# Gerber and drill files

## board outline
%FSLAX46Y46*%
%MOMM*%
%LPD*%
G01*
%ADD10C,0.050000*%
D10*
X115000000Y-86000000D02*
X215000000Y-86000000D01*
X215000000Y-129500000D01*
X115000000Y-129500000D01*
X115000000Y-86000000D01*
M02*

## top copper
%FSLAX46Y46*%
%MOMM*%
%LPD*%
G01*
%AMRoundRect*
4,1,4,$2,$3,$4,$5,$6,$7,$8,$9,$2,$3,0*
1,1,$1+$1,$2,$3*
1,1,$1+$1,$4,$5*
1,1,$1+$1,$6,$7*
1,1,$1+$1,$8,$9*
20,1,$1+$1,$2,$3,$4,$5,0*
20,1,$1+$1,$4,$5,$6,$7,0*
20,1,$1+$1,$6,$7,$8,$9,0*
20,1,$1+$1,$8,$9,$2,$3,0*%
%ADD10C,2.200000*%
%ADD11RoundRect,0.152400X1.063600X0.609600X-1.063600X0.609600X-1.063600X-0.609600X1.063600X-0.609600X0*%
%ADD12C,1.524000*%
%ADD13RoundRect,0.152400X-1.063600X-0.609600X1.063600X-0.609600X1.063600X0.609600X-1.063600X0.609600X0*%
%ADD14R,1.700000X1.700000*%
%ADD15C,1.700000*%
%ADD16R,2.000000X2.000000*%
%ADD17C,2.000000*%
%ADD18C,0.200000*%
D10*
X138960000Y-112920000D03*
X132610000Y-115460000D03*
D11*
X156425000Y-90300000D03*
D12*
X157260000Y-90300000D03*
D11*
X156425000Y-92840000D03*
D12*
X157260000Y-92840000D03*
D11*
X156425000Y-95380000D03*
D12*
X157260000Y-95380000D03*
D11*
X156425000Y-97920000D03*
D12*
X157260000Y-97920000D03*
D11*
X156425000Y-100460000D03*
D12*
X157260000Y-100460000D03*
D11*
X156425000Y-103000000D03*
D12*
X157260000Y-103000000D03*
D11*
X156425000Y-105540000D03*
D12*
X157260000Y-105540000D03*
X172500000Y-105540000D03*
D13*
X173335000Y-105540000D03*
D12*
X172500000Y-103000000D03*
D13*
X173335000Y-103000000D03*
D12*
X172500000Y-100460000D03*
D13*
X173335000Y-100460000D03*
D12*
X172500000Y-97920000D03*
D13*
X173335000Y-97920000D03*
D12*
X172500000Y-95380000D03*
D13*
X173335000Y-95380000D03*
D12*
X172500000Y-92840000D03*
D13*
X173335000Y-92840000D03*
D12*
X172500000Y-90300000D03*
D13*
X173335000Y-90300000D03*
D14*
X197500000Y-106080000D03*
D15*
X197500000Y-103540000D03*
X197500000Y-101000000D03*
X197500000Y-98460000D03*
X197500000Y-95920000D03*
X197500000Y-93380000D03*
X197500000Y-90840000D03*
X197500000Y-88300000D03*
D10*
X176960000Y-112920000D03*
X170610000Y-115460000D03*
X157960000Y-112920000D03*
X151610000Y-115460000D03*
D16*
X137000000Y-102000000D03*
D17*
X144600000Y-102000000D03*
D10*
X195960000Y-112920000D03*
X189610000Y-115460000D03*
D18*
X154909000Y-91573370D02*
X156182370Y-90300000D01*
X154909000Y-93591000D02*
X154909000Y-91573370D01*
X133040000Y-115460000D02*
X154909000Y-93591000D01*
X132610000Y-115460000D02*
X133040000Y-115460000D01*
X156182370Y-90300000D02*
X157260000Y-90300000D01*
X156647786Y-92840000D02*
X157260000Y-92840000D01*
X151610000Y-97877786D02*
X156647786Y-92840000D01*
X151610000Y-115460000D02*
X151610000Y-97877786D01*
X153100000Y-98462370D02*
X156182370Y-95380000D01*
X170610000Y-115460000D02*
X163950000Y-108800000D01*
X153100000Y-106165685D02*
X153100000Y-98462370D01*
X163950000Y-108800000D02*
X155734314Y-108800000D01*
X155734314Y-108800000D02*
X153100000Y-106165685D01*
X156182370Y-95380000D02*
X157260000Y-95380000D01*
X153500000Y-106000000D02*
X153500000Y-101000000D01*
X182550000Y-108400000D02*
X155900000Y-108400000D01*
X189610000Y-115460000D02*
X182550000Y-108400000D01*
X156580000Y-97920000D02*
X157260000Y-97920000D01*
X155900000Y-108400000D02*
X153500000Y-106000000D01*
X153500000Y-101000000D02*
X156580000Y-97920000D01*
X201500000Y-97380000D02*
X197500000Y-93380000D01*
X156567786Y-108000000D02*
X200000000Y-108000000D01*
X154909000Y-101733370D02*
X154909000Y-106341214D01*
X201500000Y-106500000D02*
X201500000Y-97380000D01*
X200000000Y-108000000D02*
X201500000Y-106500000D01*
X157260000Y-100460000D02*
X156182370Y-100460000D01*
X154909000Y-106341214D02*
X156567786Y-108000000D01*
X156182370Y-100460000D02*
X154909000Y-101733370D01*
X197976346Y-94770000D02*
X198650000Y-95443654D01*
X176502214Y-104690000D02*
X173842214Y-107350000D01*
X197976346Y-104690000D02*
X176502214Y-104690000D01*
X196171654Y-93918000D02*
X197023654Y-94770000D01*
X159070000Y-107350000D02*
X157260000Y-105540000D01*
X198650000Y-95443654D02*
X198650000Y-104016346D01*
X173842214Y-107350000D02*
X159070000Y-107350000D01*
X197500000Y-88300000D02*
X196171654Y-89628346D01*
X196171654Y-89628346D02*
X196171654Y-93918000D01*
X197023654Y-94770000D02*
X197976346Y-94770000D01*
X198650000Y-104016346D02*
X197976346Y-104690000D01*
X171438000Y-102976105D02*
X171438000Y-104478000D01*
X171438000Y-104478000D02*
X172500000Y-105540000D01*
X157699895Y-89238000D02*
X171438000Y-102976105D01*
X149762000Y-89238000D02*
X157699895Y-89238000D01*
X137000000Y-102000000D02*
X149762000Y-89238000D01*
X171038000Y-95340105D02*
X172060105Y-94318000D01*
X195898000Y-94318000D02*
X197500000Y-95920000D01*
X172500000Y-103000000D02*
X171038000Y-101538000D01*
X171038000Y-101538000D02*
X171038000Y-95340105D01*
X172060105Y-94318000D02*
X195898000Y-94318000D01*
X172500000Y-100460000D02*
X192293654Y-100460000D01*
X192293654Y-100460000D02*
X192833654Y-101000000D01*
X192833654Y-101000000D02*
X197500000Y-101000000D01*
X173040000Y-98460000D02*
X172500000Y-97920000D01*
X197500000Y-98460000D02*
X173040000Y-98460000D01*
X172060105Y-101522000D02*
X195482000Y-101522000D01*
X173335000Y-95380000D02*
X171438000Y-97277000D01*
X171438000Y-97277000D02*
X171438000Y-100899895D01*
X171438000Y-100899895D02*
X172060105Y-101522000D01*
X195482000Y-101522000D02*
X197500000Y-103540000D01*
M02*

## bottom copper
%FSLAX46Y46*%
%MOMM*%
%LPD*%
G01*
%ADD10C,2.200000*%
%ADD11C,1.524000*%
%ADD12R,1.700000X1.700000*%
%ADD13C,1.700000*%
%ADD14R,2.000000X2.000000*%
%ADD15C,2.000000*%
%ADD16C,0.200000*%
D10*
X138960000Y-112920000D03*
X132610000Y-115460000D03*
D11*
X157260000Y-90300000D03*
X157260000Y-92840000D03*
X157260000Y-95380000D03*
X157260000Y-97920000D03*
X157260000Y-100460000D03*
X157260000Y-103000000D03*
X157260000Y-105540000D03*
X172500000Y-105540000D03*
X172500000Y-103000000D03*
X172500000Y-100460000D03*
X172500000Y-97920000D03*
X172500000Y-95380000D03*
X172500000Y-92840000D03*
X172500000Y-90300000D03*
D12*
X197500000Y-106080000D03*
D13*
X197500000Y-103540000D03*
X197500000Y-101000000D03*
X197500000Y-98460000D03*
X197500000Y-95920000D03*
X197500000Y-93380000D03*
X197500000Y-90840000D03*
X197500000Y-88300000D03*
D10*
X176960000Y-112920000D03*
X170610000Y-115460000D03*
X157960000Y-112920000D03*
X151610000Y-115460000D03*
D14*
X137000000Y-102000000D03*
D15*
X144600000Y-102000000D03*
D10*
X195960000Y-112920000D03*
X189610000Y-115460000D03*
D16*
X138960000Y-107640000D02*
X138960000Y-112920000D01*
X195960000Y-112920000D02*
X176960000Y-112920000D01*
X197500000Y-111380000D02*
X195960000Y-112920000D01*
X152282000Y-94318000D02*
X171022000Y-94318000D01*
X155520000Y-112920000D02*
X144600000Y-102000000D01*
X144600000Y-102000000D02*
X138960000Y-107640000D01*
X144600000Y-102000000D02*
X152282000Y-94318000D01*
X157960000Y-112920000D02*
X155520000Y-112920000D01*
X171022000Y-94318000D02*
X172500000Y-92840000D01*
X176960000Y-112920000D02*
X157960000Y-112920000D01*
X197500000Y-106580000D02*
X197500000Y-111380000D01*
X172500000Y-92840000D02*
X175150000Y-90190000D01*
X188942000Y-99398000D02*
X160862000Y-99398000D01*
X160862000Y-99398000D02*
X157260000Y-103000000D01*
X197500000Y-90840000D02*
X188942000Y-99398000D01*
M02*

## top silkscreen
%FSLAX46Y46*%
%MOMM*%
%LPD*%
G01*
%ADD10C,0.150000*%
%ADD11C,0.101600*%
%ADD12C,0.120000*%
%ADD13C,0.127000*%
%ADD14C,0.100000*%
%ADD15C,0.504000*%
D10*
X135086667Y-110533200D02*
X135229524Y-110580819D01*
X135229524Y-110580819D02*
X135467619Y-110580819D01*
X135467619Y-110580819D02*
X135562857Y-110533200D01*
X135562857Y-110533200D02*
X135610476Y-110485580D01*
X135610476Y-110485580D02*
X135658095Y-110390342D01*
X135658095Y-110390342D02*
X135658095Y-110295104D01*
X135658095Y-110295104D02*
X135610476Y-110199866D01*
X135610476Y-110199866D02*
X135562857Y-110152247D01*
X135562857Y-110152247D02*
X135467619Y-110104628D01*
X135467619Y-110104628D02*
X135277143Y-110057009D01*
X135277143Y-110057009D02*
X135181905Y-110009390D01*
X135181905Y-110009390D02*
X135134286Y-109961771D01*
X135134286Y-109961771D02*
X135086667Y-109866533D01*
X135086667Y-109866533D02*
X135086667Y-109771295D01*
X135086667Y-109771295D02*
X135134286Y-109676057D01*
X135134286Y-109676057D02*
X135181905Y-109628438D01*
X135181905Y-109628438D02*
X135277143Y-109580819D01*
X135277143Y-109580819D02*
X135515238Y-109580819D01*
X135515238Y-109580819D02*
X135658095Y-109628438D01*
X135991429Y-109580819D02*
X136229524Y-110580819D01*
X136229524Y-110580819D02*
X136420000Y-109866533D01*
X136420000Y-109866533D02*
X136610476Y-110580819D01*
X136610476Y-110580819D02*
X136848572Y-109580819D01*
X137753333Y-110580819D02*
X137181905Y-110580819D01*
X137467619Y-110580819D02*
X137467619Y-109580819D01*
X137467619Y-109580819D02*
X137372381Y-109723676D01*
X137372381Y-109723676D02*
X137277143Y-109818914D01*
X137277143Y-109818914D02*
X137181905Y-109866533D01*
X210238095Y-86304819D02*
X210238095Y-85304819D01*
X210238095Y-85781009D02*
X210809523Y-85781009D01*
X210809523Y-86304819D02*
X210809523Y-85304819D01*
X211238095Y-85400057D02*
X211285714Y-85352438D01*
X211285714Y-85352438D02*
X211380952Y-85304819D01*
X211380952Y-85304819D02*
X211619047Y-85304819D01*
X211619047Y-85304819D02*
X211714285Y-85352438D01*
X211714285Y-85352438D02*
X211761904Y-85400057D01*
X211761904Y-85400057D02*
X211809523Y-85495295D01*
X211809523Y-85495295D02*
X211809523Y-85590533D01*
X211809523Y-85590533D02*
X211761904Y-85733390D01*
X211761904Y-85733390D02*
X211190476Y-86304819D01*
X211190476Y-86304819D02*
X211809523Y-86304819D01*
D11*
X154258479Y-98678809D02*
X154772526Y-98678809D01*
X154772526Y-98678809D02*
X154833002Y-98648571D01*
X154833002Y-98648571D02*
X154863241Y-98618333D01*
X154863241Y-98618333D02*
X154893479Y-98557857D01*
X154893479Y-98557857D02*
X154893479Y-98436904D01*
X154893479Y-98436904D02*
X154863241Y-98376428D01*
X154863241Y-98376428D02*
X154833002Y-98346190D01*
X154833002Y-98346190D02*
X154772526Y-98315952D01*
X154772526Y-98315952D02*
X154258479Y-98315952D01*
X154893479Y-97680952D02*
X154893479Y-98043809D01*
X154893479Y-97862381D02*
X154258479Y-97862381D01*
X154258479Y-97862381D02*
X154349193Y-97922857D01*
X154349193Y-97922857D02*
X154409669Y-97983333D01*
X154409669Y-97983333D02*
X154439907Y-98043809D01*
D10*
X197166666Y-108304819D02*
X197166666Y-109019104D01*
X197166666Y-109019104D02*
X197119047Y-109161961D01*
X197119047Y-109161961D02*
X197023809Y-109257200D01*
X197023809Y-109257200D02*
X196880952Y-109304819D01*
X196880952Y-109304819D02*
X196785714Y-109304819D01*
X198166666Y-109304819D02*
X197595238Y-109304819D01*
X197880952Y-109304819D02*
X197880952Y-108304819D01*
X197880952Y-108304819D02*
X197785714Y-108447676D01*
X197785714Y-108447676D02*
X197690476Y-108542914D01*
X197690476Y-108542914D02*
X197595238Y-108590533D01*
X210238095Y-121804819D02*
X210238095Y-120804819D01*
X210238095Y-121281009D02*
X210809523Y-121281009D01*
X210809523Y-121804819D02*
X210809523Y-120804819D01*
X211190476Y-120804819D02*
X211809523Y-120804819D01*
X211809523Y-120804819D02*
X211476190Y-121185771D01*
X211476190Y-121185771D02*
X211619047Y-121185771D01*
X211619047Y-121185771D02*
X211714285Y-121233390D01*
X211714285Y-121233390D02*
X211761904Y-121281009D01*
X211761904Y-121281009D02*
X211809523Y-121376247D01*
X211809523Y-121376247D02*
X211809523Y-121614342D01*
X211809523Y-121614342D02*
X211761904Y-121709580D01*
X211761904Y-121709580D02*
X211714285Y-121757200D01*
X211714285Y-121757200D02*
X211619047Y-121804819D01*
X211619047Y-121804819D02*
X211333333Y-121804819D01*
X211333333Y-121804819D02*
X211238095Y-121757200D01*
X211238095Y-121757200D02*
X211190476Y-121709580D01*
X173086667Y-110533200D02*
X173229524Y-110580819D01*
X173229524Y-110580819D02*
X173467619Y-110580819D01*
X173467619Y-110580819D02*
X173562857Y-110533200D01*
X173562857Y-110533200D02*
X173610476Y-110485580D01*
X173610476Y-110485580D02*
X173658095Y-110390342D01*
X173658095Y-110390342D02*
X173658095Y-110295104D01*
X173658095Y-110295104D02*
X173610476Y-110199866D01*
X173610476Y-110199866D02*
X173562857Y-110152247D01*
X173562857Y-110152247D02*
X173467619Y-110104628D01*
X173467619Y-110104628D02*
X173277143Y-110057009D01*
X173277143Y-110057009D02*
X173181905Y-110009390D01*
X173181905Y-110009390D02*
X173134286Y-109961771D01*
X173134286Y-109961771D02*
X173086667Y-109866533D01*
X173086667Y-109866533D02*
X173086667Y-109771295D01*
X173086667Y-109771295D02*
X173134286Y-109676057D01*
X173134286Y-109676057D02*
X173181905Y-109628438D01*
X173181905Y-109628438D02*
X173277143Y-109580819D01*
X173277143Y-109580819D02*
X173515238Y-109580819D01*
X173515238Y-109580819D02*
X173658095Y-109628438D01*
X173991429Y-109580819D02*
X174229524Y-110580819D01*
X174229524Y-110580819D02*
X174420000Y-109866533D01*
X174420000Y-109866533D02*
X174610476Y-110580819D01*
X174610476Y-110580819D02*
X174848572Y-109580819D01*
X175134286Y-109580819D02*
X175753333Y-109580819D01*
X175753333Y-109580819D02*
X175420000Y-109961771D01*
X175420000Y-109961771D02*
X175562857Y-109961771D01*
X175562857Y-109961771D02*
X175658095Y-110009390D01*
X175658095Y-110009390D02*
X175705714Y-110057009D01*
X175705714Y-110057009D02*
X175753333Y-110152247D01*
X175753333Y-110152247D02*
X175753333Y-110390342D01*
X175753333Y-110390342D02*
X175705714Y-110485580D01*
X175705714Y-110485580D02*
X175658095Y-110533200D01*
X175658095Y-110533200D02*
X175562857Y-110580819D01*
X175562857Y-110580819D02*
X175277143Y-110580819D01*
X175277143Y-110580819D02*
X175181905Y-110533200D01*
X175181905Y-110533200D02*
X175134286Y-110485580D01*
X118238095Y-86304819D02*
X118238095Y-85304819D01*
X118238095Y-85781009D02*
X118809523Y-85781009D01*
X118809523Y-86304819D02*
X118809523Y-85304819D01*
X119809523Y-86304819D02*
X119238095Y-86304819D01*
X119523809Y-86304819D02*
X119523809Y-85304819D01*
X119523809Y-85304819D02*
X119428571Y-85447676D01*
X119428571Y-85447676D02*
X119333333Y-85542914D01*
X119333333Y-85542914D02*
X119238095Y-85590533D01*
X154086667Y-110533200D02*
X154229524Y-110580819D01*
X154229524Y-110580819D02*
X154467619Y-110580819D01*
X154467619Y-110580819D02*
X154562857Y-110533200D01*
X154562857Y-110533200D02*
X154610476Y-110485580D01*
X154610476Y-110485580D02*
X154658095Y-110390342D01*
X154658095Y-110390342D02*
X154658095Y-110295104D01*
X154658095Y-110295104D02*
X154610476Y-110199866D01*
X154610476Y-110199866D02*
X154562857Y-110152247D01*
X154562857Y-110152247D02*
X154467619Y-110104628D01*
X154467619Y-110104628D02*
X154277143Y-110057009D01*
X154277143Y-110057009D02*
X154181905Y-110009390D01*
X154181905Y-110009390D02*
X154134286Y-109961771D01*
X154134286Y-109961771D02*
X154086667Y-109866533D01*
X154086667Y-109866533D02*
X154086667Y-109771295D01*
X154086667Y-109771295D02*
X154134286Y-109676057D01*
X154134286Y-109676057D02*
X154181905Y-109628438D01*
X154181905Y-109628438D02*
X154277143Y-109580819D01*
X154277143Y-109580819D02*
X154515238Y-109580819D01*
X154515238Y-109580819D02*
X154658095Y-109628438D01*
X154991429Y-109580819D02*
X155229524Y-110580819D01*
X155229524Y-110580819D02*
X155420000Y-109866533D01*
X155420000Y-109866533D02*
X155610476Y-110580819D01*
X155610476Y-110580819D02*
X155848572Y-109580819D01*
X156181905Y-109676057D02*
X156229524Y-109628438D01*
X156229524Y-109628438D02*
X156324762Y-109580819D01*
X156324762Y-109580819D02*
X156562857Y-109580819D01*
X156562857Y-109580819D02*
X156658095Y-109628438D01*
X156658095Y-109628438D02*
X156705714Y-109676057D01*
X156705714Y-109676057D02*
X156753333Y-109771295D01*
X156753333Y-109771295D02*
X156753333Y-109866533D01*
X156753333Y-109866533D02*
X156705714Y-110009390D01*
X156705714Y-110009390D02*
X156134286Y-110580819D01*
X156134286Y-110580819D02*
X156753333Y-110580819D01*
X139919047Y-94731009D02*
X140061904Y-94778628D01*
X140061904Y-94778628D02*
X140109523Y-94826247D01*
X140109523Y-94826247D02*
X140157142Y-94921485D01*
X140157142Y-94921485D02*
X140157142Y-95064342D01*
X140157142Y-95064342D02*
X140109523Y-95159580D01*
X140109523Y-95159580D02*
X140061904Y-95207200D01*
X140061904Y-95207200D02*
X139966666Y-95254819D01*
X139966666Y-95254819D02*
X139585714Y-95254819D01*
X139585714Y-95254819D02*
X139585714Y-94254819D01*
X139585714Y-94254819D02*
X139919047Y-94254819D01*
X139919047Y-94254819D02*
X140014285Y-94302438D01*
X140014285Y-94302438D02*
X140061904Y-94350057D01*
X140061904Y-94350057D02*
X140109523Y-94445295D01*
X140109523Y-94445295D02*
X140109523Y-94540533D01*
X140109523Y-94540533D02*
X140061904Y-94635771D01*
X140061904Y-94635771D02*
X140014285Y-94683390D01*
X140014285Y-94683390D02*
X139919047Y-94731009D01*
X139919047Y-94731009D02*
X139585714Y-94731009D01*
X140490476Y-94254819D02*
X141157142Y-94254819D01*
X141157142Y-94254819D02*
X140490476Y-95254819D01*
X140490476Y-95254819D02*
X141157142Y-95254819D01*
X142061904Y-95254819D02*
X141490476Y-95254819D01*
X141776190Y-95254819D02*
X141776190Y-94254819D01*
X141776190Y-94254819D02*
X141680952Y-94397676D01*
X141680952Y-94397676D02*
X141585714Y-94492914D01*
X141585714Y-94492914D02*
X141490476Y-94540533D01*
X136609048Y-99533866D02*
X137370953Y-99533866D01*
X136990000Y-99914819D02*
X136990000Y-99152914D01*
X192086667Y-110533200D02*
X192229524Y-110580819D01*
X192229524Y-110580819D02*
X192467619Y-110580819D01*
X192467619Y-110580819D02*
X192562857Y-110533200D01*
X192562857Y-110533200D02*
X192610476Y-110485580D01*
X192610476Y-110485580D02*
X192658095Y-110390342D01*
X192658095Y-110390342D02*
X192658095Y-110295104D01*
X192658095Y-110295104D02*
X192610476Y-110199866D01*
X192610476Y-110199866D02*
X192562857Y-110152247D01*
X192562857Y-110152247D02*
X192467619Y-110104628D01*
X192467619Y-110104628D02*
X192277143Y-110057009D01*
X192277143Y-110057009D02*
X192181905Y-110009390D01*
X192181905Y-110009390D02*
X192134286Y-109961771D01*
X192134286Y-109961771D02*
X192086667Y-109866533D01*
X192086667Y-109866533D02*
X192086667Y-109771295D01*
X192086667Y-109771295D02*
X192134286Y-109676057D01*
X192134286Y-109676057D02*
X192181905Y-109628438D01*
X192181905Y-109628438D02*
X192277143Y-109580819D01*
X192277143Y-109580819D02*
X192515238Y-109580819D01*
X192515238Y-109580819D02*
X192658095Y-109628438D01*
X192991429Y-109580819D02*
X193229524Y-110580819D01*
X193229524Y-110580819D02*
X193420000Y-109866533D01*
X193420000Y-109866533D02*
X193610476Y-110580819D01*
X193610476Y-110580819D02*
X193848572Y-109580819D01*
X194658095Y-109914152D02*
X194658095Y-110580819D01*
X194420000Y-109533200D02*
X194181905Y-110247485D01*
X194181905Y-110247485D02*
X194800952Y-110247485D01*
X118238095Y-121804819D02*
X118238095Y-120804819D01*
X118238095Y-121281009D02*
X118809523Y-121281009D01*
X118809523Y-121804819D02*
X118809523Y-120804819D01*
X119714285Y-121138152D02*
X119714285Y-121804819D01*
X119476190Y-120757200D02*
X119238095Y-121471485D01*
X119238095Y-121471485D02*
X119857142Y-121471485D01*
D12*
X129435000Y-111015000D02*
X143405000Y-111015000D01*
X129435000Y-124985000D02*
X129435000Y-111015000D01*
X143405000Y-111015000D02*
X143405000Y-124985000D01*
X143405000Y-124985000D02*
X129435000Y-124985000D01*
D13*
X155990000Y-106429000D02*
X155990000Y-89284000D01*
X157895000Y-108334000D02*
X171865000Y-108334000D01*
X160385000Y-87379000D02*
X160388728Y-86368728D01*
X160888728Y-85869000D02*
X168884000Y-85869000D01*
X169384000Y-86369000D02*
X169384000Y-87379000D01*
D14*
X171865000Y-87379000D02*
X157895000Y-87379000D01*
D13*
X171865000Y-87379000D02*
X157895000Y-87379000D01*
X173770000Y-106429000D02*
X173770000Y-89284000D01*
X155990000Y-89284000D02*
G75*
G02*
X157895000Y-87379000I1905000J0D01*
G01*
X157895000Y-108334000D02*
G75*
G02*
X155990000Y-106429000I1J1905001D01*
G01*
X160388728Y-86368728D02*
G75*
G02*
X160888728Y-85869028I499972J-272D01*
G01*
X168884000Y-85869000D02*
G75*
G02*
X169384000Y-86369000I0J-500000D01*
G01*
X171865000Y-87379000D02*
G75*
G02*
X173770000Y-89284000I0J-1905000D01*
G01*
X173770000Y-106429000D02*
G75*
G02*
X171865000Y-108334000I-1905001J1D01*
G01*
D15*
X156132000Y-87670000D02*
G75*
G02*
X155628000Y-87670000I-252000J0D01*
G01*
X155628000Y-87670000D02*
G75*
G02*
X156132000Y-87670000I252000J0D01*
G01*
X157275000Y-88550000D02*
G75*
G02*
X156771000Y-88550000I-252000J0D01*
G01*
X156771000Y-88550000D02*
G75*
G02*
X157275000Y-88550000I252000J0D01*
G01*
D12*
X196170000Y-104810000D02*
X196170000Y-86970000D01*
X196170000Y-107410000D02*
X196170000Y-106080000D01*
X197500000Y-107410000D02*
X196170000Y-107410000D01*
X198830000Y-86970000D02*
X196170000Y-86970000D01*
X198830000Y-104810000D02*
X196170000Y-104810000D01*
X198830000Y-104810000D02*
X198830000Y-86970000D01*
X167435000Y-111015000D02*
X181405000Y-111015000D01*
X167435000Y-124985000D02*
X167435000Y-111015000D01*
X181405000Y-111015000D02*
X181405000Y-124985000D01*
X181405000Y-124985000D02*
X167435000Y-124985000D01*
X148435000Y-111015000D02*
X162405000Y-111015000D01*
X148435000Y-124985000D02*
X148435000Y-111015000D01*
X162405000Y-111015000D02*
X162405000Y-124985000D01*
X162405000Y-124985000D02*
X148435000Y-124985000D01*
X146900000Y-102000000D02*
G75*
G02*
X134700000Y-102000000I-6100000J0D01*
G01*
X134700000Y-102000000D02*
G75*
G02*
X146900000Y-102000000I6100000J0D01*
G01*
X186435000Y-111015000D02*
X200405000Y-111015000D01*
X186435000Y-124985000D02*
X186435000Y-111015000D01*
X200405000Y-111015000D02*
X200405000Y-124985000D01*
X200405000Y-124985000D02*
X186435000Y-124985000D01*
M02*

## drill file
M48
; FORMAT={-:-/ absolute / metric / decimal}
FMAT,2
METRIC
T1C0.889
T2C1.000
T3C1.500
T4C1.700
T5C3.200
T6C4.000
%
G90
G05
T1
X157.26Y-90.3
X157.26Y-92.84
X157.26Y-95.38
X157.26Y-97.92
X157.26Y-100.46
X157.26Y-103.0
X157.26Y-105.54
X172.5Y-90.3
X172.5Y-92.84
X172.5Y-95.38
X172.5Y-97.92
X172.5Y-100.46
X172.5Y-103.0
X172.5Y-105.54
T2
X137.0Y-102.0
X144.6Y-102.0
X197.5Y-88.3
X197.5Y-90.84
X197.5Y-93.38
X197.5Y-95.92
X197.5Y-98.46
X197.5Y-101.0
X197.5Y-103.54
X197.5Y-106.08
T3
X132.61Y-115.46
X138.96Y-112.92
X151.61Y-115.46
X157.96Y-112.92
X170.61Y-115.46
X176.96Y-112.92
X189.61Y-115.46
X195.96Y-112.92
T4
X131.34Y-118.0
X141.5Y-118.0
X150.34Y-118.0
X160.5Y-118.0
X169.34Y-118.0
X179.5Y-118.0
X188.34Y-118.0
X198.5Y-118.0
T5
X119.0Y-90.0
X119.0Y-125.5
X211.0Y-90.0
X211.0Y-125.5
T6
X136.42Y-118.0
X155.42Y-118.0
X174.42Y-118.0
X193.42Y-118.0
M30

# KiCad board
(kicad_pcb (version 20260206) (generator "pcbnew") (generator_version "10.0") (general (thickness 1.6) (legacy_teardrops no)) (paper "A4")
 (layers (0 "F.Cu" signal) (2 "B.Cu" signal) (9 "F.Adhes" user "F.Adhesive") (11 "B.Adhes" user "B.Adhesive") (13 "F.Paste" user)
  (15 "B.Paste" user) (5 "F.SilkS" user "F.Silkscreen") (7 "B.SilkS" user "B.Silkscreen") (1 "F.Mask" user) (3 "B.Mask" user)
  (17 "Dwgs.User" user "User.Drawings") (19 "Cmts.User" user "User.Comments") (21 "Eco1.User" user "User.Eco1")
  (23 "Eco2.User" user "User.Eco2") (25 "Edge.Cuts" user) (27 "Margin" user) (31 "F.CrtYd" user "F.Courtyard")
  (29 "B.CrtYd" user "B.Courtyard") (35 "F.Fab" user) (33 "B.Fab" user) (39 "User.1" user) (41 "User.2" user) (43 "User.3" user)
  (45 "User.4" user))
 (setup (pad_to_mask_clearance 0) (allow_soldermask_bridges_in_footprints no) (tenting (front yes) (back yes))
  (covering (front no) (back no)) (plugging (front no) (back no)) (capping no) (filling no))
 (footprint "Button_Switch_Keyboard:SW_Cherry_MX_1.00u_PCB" (layer "F.Cu") (at 138.96 112.92)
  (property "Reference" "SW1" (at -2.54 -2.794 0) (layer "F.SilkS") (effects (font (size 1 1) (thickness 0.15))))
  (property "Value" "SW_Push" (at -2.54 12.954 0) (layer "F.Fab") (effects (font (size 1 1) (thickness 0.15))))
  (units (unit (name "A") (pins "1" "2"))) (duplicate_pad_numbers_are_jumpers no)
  (fp_line (start -9.525 -1.905) (end 4.445 -1.905) (stroke (width 0.12) (type solid)) (layer "F.SilkS"))
  (fp_line (start -9.525 12.065) (end -9.525 -1.905) (stroke (width 0.12) (type solid)) (layer "F.SilkS"))
  (fp_line (start 4.445 -1.905) (end 4.445 12.065) (stroke (width 0.12) (type solid)) (layer "F.SilkS"))
  (fp_line (start 4.445 12.065) (end -9.525 12.065) (stroke (width 0.12) (type solid)) (layer "F.SilkS"))
  (pad "" np_thru_hole circle (at -7.62 5.08) (size 1.7 1.7) (drill 1.7) (layers "*.Cu" "*.Mask"))
  (pad "" np_thru_hole circle (at -2.54 5.08) (size 4 4) (drill 4) (layers "*.Cu" "*.Mask"))
  (pad "" np_thru_hole circle (at 2.54 5.08) (size 1.7 1.7) (drill 1.7) (layers "*.Cu" "*.Mask"))
  (pad "1" thru_hole circle (at 0 0) (size 2.2 2.2) (drill 1.5) (layers "*.Cu" "*.Mask") (remove_unused_layers no) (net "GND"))
  (pad "2" thru_hole circle (at -6.35 2.54) (size 2.2 2.2) (drill 1.5) (layers "*.Cu" "*.Mask") (remove_unused_layers no)
   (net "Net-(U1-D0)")))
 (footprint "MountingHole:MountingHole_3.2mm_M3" (layer "F.Cu") (at 211 90)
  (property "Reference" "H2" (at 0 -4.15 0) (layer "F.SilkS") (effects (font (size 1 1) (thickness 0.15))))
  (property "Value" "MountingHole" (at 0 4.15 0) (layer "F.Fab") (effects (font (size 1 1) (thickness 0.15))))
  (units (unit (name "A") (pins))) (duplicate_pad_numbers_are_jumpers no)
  (pad "" np_thru_hole circle (at 0 0) (size 3.2 3.2) (drill 3.2) (layers "*.Cu" "*.Mask")))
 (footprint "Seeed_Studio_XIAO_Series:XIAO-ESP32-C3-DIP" (layer "F.Cu") (at 164.88 97.92 90)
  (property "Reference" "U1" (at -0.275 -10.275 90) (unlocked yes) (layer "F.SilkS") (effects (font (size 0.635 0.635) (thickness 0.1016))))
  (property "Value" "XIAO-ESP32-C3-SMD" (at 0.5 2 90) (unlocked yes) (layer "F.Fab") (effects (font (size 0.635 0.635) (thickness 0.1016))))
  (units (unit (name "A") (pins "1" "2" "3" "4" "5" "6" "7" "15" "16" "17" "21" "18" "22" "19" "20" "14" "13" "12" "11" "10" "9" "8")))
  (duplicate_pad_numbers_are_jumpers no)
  (fp_line (start -8.509 -8.89) (end 8.636 -8.89) (stroke (width 0.127) (type solid)) (layer "F.SilkS"))
  (fp_line (start -10.414 -6.985) (end -10.414 6.985) (stroke (width 0.127) (type solid)) (layer "F.SilkS"))
  (fp_line (start 10.541 -4.495) (end 11.551272 -4.491272) (stroke (width 0.127) (type solid)) (layer "F.SilkS"))
  (fp_line (start 12.051 -3.991272) (end 12.051 4.004) (stroke (width 0.127) (type solid)) (layer "F.SilkS"))
  (fp_line (start 11.551 4.504) (end 10.541 4.504) (stroke (width 0.127) (type solid)) (layer "F.SilkS"))
  (fp_line (start 10.541 6.985) (end 10.541 -6.985) (stroke (width 0.1) (type solid)) (layer "F.SilkS"))
  (fp_line (start 10.541 6.985) (end 10.541 -6.985) (stroke (width 0.127) (type solid)) (layer "F.SilkS"))
  (fp_line (start -8.509 8.89) (end 8.636 8.89) (stroke (width 0.127) (type solid)) (layer "F.SilkS"))
  (fp_arc (start 8.636 -8.89) (mid 9.983038 -8.332038) (end 10.541 -6.985) (stroke (width 0.127) (type solid)) (layer "F.SilkS"))
  (fp_arc (start -10.414 -6.985) (mid -9.856038 -8.332038) (end -8.509 -8.89) (stroke (width 0.127) (type solid)) (layer "F.SilkS"))
  (fp_arc (start 11.551272 -4.491272) (mid 11.90464 -4.344728) (end 12.051 -3.991272) (stroke (width 0.127) (type default))
   (layer "F.SilkS"))
  (fp_arc (start 12.051 4.004) (mid 11.904553 4.357553) (end 11.551 4.504) (stroke (width 0.127) (type default)) (layer "F.SilkS"))
  (fp_arc (start 10.541 6.985) (mid 9.983038 8.332038) (end 8.636 8.89) (stroke (width 0.127) (type solid)) (layer "F.SilkS"))
  (fp_arc (start -8.509 8.89) (mid -9.856038 8.332038) (end -10.414 6.985) (stroke (width 0.127) (type solid)) (layer "F.SilkS"))
  (fp_circle (center 10.25 -9) (end 10.504 -9) (stroke (width 0.5) (type solid)) (fill yes) (layer "F.SilkS"))
  (fp_circle (center 9.37 -7.857) (end 9.624 -7.857) (stroke (width 0.5) (type solid)) (fill yes) (layer "F.SilkS"))
  (pad "1" smd roundrect (at 7.62 -8.455 180) (size 2.432 1.524) (layers "F.Cu" "F.Mask") (roundrect_rratio 0.1) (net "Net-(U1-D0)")
   (thermal_bridge_angle 45))
  (pad "1" thru_hole circle (at 7.62 -7.62 180) (size 1.524 1.524) (drill 0.889) (layers "*.Cu" "*.Mask") (remove_unused_layers no)
   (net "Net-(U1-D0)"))
  (pad "2" smd roundrect (at 5.08 -8.455 180) (size 2.432 1.524) (layers "F.Cu" "F.Mask") (roundrect_rratio 0.1) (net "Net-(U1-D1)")
   (thermal_bridge_angle 45))
  (pad "2" thru_hole circle (at 5.08 -7.62 180) (size 1.524 1.524) (drill 0.889) (layers "*.Cu" "*.Mask") (remove_unused_layers no)
   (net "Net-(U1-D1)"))
  (pad "3" smd roundrect (at 2.54 -8.455 180) (size 2.432 1.524) (layers "F.Cu" "F.Mask") (roundrect_rratio 0.1) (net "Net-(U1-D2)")
   (thermal_bridge_angle 45))
  (pad "3" thru_hole circle (at 2.54 -7.62 180) (size 1.524 1.524) (drill 0.889) (layers "*.Cu" "*.Mask") (remove_unused_layers no)
   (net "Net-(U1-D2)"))
  (pad "4" smd roundrect (at 0 -8.455 180) (size 2.432 1.524) (layers "F.Cu" "F.Mask") (roundrect_rratio 0.1) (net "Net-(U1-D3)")
   (thermal_bridge_angle 45))
  (pad "4" thru_hole circle (at 0 -7.62 180) (size 1.524 1.524) (drill 0.889) (layers "*.Cu" "*.Mask") (remove_unused_layers no)
   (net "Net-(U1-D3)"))
  (pad "5" smd roundrect (at -2.54 -8.455 180) (size 2.432 1.524) (layers "F.Cu" "F.Mask") (roundrect_rratio 0.1) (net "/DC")
   (thermal_bridge_angle 45))
  (pad "5" thru_hole circle (at -2.54 -7.62 180) (size 1.524 1.524) (drill 0.889) (layers "*.Cu" "*.Mask") (remove_unused_layers no)
   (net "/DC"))
  (pad "6" smd roundrect (at -5.08 -8.455 180) (size 2.432 1.524) (layers "F.Cu" "F.Mask") (roundrect_rratio 0.1) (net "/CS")
   (thermal_bridge_angle 45))
  (pad "6" thru_hole circle (at -5.08 -7.62 180) (size 1.524 1.524) (drill 0.889) (layers "*.Cu" "*.Mask") (remove_unused_layers no)
   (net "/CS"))
  (pad "7" smd roundrect (at -7.62 -8.455 180) (size 2.432 1.524) (layers "F.Cu" "F.Mask") (roundrect_rratio 0.1) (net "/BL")
   (thermal_bridge_angle 45))
  (pad "7" thru_hole circle (at -7.62 -7.62 180) (size 1.524 1.524) (drill 0.889) (layers "*.Cu" "*.Mask") (remove_unused_layers no)
   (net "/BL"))
  (pad "8" thru_hole circle (at -7.62 7.62) (size 1.524 1.524) (drill 0.889) (layers "*.Cu" "*.Mask") (remove_unused_layers no)
   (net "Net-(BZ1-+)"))
  (pad "8" smd roundrect (at -7.62 8.455) (size 2.432 1.524) (layers "F.Cu" "F.Mask") (roundrect_rratio 0.1) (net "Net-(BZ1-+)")
   (thermal_bridge_angle 45))
  (pad "9" thru_hole circle (at -5.08 7.62) (size 1.524 1.524) (drill 0.889) (layers "*.Cu" "*.Mask") (remove_unused_layers no) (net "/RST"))
  (pad "9" smd roundrect (at -5.08 8.455) (size 2.432 1.524) (layers "F.Cu" "F.Mask") (roundrect_rratio 0.1) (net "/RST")
   (thermal_bridge_angle 45))
  (pad "10" thru_hole circle (at -2.54 7.62) (size 1.524 1.524) (drill 0.889) (layers "*.Cu" "*.Mask") (remove_unused_layers no)
   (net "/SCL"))
  (pad "10" smd roundrect (at -2.54 8.455) (size 2.432 1.524) (layers "F.Cu" "F.Mask") (roundrect_rratio 0.1) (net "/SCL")
   (thermal_bridge_angle 45))
  (pad "11" thru_hole circle (at 0 7.62) (size 1.524 1.524) (drill 0.889) (layers "*.Cu" "*.Mask") (remove_unused_layers no) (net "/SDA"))
  (pad "11" smd roundrect (at 0 8.455) (size 2.432 1.524) (layers "F.Cu" "F.Mask") (roundrect_rratio 0.1) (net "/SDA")
   (thermal_bridge_angle 45))
  (pad "12" thru_hole circle (at 2.54 7.62) (size 1.524 1.524) (drill 0.889) (layers "*.Cu" "*.Mask") (remove_unused_layers no)
   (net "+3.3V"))
  (pad "12" smd roundrect (at 2.54 8.455) (size 2.432 1.524) (layers "F.Cu" "F.Mask") (roundrect_rratio 0.1) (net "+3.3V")
   (thermal_bridge_angle 45))
  (pad "13" thru_hole circle (at 5.08 7.62) (size 1.524 1.524) (drill 0.889) (layers "*.Cu" "*.Mask") (remove_unused_layers no) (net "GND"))
  (pad "13" smd roundrect (at 5.08 8.455) (size 2.432 1.524) (layers "F.Cu" "F.Mask") (roundrect_rratio 0.1) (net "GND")
   (thermal_bridge_angle 45))
  (pad "14" thru_hole circle (at 7.62 7.62) (size 1.524 1.524) (drill 0.889) (layers "*.Cu" "*.Mask") (remove_unused_layers no)
   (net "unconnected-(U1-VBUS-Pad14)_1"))
  (pad "14" smd roundrect (at 7.62 8.455) (size 2.432 1.524) (layers "F.Cu" "F.Mask") (roundrect_rratio 0.1)
   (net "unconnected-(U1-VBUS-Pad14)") (thermal_bridge_angle 45)))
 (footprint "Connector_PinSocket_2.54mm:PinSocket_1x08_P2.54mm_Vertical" (layer "F.Cu") (at 197.5 106.08 180)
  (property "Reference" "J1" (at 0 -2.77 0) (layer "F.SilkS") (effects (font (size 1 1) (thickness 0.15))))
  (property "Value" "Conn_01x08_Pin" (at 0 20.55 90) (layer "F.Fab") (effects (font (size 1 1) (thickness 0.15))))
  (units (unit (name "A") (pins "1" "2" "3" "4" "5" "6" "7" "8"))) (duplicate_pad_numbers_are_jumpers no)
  (fp_line (start 1.33 1.27) (end 1.33 19.11) (stroke (width 0.12) (type solid)) (layer "F.SilkS"))
  (fp_line (start 1.33 -1.33) (end 1.33 0) (stroke (width 0.12) (type solid)) (layer "F.SilkS"))
  (fp_line (start 0 -1.33) (end 1.33 -1.33) (stroke (width 0.12) (type solid)) (layer "F.SilkS"))
  (fp_line (start -1.33 19.11) (end 1.33 19.11) (stroke (width 0.12) (type solid)) (layer "F.SilkS"))
  (fp_line (start -1.33 1.27) (end 1.33 1.27) (stroke (width 0.12) (type solid)) (layer "F.SilkS"))
  (fp_line (start -1.33 1.27) (end -1.33 19.11) (stroke (width 0.12) (type solid)) (layer "F.SilkS"))
  (pad "1" thru_hole rect (at 0 0 180) (size 1.7 1.7) (drill 1) (layers "*.Cu" "*.Mask") (remove_unused_layers no) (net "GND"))
  (pad "2" thru_hole circle (at 0 2.54 180) (size 1.7 1.7) (drill 1) (layers "*.Cu" "*.Mask") (remove_unused_layers no) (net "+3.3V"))
  (pad "3" thru_hole circle (at 0 5.08 180) (size 1.7 1.7) (drill 1) (layers "*.Cu" "*.Mask") (remove_unused_layers no) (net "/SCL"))
  (pad "4" thru_hole circle (at 0 7.62 180) (size 1.7 1.7) (drill 1) (layers "*.Cu" "*.Mask") (remove_unused_layers no) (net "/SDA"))
  (pad "5" thru_hole circle (at 0 10.16 180) (size 1.7 1.7) (drill 1) (layers "*.Cu" "*.Mask") (remove_unused_layers no) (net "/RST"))
  (pad "6" thru_hole circle (at 0 12.7 180) (size 1.7 1.7) (drill 1) (layers "*.Cu" "*.Mask") (remove_unused_layers no) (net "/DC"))
  (pad "7" thru_hole circle (at 0 15.24 180) (size 1.7 1.7) (drill 1) (layers "*.Cu" "*.Mask") (remove_unused_layers no) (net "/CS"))
  (pad "8" thru_hole circle (at 0 17.78 180) (size 1.7 1.7) (drill 1) (layers "*.Cu" "*.Mask") (remove_unused_layers no) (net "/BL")))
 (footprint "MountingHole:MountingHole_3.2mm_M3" (layer "F.Cu") (at 211 125.5)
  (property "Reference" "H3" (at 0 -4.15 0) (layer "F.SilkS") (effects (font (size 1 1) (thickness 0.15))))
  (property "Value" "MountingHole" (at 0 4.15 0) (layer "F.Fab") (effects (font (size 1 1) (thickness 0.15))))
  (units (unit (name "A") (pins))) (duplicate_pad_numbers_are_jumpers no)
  (pad "" np_thru_hole circle (at 0 0) (size 3.2 3.2) (drill 3.2) (layers "*.Cu" "*.Mask")))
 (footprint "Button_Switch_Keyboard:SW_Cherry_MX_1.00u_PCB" (layer "F.Cu") (at 176.96 112.92)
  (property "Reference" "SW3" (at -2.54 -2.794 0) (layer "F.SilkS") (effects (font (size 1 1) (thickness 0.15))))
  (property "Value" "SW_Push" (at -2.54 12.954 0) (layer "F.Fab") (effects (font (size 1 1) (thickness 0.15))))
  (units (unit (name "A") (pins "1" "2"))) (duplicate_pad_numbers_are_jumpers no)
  (fp_line (start -9.525 -1.905) (end 4.445 -1.905) (stroke (width 0.12) (type solid)) (layer "F.SilkS"))
  (fp_line (start -9.525 12.065) (end -9.525 -1.905) (stroke (width 0.12) (type solid)) (layer "F.SilkS"))
  (fp_line (start 4.445 -1.905) (end 4.445 12.065) (stroke (width 0.12) (type solid)) (layer "F.SilkS"))
  (fp_line (start 4.445 12.065) (end -9.525 12.065) (stroke (width 0.12) (type solid)) (layer "F.SilkS"))
  (pad "" np_thru_hole circle (at -7.62 5.08) (size 1.7 1.7) (drill 1.7) (layers "*.Cu" "*.Mask"))
  (pad "" np_thru_hole circle (at -2.54 5.08) (size 4 4) (drill 4) (layers "*.Cu" "*.Mask"))
  (pad "" np_thru_hole circle (at 2.54 5.08) (size 1.7 1.7) (drill 1.7) (layers "*.Cu" "*.Mask"))
  (pad "1" thru_hole circle (at 0 0) (size 2.2 2.2) (drill 1.5) (layers "*.Cu" "*.Mask") (remove_unused_layers no) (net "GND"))
  (pad "2" thru_hole circle (at -6.35 2.54) (size 2.2 2.2) (drill 1.5) (layers "*.Cu" "*.Mask") (remove_unused_layers no)
   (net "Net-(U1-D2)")))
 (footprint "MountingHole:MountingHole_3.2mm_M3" (layer "F.Cu") (at 119 90)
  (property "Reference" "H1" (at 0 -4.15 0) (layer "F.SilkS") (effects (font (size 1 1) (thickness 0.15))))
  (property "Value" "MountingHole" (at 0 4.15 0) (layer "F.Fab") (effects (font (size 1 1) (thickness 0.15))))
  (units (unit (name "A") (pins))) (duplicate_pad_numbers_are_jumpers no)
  (pad "" np_thru_hole circle (at 0 0) (size 3.2 3.2) (drill 3.2) (layers "*.Cu" "*.Mask")))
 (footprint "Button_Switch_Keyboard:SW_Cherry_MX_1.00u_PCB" (layer "F.Cu") (at 157.96 112.92)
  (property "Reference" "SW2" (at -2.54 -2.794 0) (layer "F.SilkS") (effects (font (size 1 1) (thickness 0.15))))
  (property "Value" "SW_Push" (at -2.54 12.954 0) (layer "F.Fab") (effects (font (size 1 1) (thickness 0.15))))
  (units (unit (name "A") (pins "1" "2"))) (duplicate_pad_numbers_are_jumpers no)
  (fp_line (start -9.525 -1.905) (end 4.445 -1.905) (stroke (width 0.12) (type solid)) (layer "F.SilkS"))
  (fp_line (start -9.525 12.065) (end -9.525 -1.905) (stroke (width 0.12) (type solid)) (layer "F.SilkS"))
  (fp_line (start 4.445 -1.905) (end 4.445 12.065) (stroke (width 0.12) (type solid)) (layer "F.SilkS"))
  (fp_line (start 4.445 12.065) (end -9.525 12.065) (stroke (width 0.12) (type solid)) (layer "F.SilkS"))
  (pad "" np_thru_hole circle (at -7.62 5.08) (size 1.7 1.7) (drill 1.7) (layers "*.Cu" "*.Mask"))
  (pad "" np_thru_hole circle (at -2.54 5.08) (size 4 4) (drill 4) (layers "*.Cu" "*.Mask"))
  (pad "" np_thru_hole circle (at 2.54 5.08) (size 1.7 1.7) (drill 1.7) (layers "*.Cu" "*.Mask"))
  (pad "1" thru_hole circle (at 0 0) (size 2.2 2.2) (drill 1.5) (layers "*.Cu" "*.Mask") (remove_unused_layers no) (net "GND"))
  (pad "2" thru_hole circle (at -6.35 2.54) (size 2.2 2.2) (drill 1.5) (layers "*.Cu" "*.Mask") (remove_unused_layers no)
   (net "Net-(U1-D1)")))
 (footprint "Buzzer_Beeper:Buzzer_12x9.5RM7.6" (layer "F.Cu") (at 137 102)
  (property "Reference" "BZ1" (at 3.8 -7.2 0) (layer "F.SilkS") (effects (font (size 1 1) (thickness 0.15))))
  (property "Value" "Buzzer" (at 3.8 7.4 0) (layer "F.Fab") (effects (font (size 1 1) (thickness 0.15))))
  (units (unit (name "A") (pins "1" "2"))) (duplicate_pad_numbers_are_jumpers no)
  (fp_circle (center 3.8 0) (end 9.9 0) (stroke (width 0.12) (type solid)) (fill no) (layer "F.SilkS"))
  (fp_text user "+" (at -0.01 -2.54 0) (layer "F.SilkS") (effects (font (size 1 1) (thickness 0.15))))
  (pad "1" thru_hole rect (at 0 0) (size 2 2) (drill 1) (layers "*.Cu" "*.Mask") (remove_unused_layers no) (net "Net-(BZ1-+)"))
  (pad "2" thru_hole circle (at 7.6 0) (size 2 2) (drill 1) (layers "*.Cu" "*.Mask") (remove_unused_layers no) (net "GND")))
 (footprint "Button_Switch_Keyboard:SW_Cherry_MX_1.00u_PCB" (layer "F.Cu") (at 195.96 112.92)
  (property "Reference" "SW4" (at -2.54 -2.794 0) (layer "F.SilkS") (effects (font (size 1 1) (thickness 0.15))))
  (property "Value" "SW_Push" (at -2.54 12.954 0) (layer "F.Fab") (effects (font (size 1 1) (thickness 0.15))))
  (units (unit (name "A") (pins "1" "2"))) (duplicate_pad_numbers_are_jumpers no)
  (fp_line (start -9.525 -1.905) (end 4.445 -1.905) (stroke (width 0.12) (type solid)) (layer "F.SilkS"))
  (fp_line (start -9.525 12.065) (end -9.525 -1.905) (stroke (width 0.12) (type solid)) (layer "F.SilkS"))
  (fp_line (start 4.445 -1.905) (end 4.445 12.065) (stroke (width 0.12) (type solid)) (layer "F.SilkS"))
  (fp_line (start 4.445 12.065) (end -9.525 12.065) (stroke (width 0.12) (type solid)) (layer "F.SilkS"))
  (pad "" np_thru_hole circle (at -7.62 5.08) (size 1.7 1.7) (drill 1.7) (layers "*.Cu" "*.Mask"))
  (pad "" np_thru_hole circle (at -2.54 5.08) (size 4 4) (drill 4) (layers "*.Cu" "*.Mask"))
  (pad "" np_thru_hole circle (at 2.54 5.08) (size 1.7 1.7) (drill 1.7) (layers "*.Cu" "*.Mask"))
  (pad "1" thru_hole circle (at 0 0) (size 2.2 2.2) (drill 1.5) (layers "*.Cu" "*.Mask") (remove_unused_layers no) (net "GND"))
  (pad "2" thru_hole circle (at -6.35 2.54) (size 2.2 2.2) (drill 1.5) (layers "*.Cu" "*.Mask") (remove_unused_layers no)
   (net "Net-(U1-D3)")))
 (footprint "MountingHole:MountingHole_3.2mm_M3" (layer "F.Cu") (at 119 125.5)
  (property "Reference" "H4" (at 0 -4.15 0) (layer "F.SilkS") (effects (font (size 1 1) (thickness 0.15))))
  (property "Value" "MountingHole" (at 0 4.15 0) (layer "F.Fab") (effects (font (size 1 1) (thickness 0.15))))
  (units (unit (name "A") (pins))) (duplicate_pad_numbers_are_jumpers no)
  (pad "" np_thru_hole circle (at 0 0) (size 3.2 3.2) (drill 3.2) (layers "*.Cu" "*.Mask")))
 (gr_rect (start 115 86) (end 215 129.5) (stroke (width 0.05) (type default)) (fill no) (layer "Edge.Cuts"))
 (segment (start 138.96 107.64) (end 138.96 112.92) (width 0.2) (layer "B.Cu") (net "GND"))
 (segment (start 195.96 112.92) (end 176.96 112.92) (width 0.2) (layer "B.Cu") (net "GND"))
 (segment (start 197.5 111.38) (end 195.96 112.92) (width 0.2) (layer "B.Cu") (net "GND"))
 (segment (start 152.282 94.318) (end 171.022 94.318) (width 0.2) (layer "B.Cu") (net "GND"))
 (segment (start 155.52 112.92) (end 144.6 102) (width 0.2) (layer "B.Cu") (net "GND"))
 (segment (start 144.6 102) (end 138.96 107.64) (width 0.2) (layer "B.Cu") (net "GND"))
 (segment (start 144.6 102) (end 152.282 94.318) (width 0.2) (layer "B.Cu") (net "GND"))
 (segment (start 157.96 112.92) (end 155.52 112.92) (width 0.2) (layer "B.Cu") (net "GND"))
 (segment (start 171.022 94.318) (end 172.5 92.84) (width 0.2) (layer "B.Cu") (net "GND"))
 (segment (start 176.96 112.92) (end 157.96 112.92) (width 0.2) (layer "B.Cu") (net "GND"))
 (segment (start 197.5 106.58) (end 197.5 111.38) (width 0.2) (layer "B.Cu") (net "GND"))
 (segment (start 172.5 92.84) (end 175.15 90.19) (width 0.2) (layer "B.Cu") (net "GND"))
 (segment (start 154.909 91.57337) (end 156.18237 90.3) (width 0.2) (layer "F.Cu") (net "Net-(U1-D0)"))
 (segment (start 154.909 93.591) (end 154.909 91.57337) (width 0.2) (layer "F.Cu") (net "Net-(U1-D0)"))
 (segment (start 133.04 115.46) (end 154.909 93.591) (width 0.2) (layer "F.Cu") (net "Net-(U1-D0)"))
 (segment (start 132.61 115.46) (end 133.04 115.46) (width 0.2) (layer "F.Cu") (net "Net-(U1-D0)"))
 (segment (start 156.18237 90.3) (end 157.26 90.3) (width 0.2) (layer "F.Cu") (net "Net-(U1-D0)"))
 (segment (start 156.647786 92.84) (end 157.26 92.84) (width 0.2) (layer "F.Cu") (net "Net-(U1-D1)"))
 (segment (start 151.61 97.877786) (end 156.647786 92.84) (width 0.2) (layer "F.Cu") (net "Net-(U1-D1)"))
 (segment (start 151.61 115.46) (end 151.61 97.877786) (width 0.2) (layer "F.Cu") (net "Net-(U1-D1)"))
 (segment (start 153.1 98.46237) (end 156.18237 95.38) (width 0.2) (layer "F.Cu") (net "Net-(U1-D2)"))
 (segment (start 170.61 115.46) (end 163.95 108.8) (width 0.2) (layer "F.Cu") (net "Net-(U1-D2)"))
 (segment (start 153.1 106.165685) (end 153.1 98.46237) (width 0.2) (layer "F.Cu") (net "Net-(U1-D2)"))
 (segment (start 163.95 108.8) (end 155.734314 108.8) (width 0.2) (layer "F.Cu") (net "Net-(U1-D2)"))
 (segment (start 155.734314 108.8) (end 153.1 106.165685) (width 0.2) (layer "F.Cu") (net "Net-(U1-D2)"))
 (segment (start 156.18237 95.38) (end 157.26 95.38) (width 0.2) (layer "F.Cu") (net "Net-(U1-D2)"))
 (segment (start 153.5 106) (end 153.5 101) (width 0.2) (layer "F.Cu") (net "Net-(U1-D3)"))
 (segment (start 182.55 108.4) (end 155.9 108.4) (width 0.2) (layer "F.Cu") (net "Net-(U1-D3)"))
 (segment (start 189.61 115.46) (end 182.55 108.4) (width 0.2) (layer "F.Cu") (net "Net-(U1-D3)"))
 (segment (start 156.58 97.92) (end 157.26 97.92) (width 0.2) (layer "F.Cu") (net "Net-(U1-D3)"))
 (segment (start 155.9 108.4) (end 153.5 106) (width 0.2) (layer "F.Cu") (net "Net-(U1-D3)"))
 (segment (start 153.5 101) (end 156.58 97.92) (width 0.2) (layer "F.Cu") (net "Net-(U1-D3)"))
 (segment (start 201.5 97.38) (end 197.5 93.38) (width 0.2) (layer "F.Cu") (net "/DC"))
 (segment (start 156.567786 108) (end 200 108) (width 0.2) (layer "F.Cu") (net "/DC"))
 (segment (start 154.909 101.73337) (end 154.909 106.341214) (width 0.2) (layer "F.Cu") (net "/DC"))
 (segment (start 201.5 106.5) (end 201.5 97.38) (width 0.2) (layer "F.Cu") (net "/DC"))
 (segment (start 200 108) (end 201.5 106.5) (width 0.2) (layer "F.Cu") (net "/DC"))
 (segment (start 157.26 100.46) (end 156.18237 100.46) (width 0.2) (layer "F.Cu") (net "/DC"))
 (segment (start 154.909 106.341214) (end 156.567786 108) (width 0.2) (layer "F.Cu") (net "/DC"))
 (segment (start 156.18237 100.46) (end 154.909 101.73337) (width 0.2) (layer "F.Cu") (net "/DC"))
 (segment (start 188.942 99.398) (end 160.862 99.398) (width 0.2) (layer "B.Cu") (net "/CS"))
 (segment (start 160.862 99.398) (end 157.26 103) (width 0.2) (layer "B.Cu") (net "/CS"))
 (segment (start 197.5 90.84) (end 188.942 99.398) (width 0.2) (layer "B.Cu") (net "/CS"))
 (segment (start 197.976346 94.77) (end 198.65 95.443654) (width 0.2) (layer "F.Cu") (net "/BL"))
 (segment (start 176.502214 104.69) (end 173.842214 107.35) (width 0.2) (layer "F.Cu") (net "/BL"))
 (segment (start 197.976346 104.69) (end 176.502214 104.69) (width 0.2) (layer "F.Cu") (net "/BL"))
 (segment (start 196.171654 93.918) (end 197.023654 94.77) (width 0.2) (layer "F.Cu") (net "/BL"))
 (segment (start 159.07 107.35) (end 157.26 105.54) (width 0.2) (layer "F.Cu") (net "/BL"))
 (segment (start 198.65 95.443654) (end 198.65 104.016346) (width 0.2) (layer "F.Cu") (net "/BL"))
 (segment (start 173.842214 107.35) (end 159.07 107.35) (width 0.2) (layer "F.Cu") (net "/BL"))
 (segment (start 197.5 88.3) (end 196.171654 89.628346) (width 0.2) (layer "F.Cu") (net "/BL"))
 (segment (start 196.171654 89.628346) (end 196.171654 93.918) (width 0.2) (layer "F.Cu") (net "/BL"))
 (segment (start 197.023654 94.77) (end 197.976346 94.77) (width 0.2) (layer "F.Cu") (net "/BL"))
 (segment (start 198.65 104.016346) (end 197.976346 104.69) (width 0.2) (layer "F.Cu") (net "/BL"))
 (segment (start 171.438 102.976105) (end 171.438 104.478) (width 0.2) (layer "F.Cu") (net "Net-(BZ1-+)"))
 (segment (start 171.438 104.478) (end 172.5 105.54) (width 0.2) (layer "F.Cu") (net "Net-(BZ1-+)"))
 (segment (start 157.699895 89.238) (end 171.438 102.976105) (width 0.2) (layer "F.Cu") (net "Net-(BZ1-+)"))
 (segment (start 149.762 89.238) (end 157.699895 89.238) (width 0.2) (layer "F.Cu") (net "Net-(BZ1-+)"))
 (segment (start 137 102) (end 149.762 89.238) (width 0.2) (layer "F.Cu") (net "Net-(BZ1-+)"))
 (segment (start 171.038 95.340105) (end 172.060105 94.318) (width 0.2) (layer "F.Cu") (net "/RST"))
 (segment (start 195.898 94.318) (end 197.5 95.92) (width 0.2) (layer "F.Cu") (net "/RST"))
 (segment (start 172.5 103) (end 171.038 101.538) (width 0.2) (layer "F.Cu") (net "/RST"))
 (segment (start 171.038 101.538) (end 171.038 95.340105) (width 0.2) (layer "F.Cu") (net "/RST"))
 (segment (start 172.060105 94.318) (end 195.898 94.318) (width 0.2) (layer "F.Cu") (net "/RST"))
 (segment (start 172.5 100.46) (end 192.293654 100.46) (width 0.2) (layer "F.Cu") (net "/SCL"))
 (segment (start 192.293654 100.46) (end 192.833654 101) (width 0.2) (layer "F.Cu") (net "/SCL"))
 (segment (start 192.833654 101) (end 197.5 101) (width 0.2) (layer "F.Cu") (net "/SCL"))
 (segment (start 173.04 98.46) (end 172.5 97.92) (width 0.2) (layer "F.Cu") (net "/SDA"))
 (segment (start 197.5 98.46) (end 173.04 98.46) (width 0.2) (layer "F.Cu") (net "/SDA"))
 (segment (start 172.060105 101.522) (end 195.482 101.522) (width 0.2) (layer "F.Cu") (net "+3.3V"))
 (segment (start 173.335 95.38) (end 171.438 97.277) (width 0.2) (layer "F.Cu") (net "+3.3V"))
 (segment (start 171.438 97.277) (end 171.438 100.899895) (width 0.2) (layer "F.Cu") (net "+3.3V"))
 (segment (start 171.438 100.899895) (end 172.060105 101.522) (width 0.2) (layer "F.Cu") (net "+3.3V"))
 (segment (start 195.482 101.522) (end 197.5 103.54) (width 0.2) (layer "F.Cu") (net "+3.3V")))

